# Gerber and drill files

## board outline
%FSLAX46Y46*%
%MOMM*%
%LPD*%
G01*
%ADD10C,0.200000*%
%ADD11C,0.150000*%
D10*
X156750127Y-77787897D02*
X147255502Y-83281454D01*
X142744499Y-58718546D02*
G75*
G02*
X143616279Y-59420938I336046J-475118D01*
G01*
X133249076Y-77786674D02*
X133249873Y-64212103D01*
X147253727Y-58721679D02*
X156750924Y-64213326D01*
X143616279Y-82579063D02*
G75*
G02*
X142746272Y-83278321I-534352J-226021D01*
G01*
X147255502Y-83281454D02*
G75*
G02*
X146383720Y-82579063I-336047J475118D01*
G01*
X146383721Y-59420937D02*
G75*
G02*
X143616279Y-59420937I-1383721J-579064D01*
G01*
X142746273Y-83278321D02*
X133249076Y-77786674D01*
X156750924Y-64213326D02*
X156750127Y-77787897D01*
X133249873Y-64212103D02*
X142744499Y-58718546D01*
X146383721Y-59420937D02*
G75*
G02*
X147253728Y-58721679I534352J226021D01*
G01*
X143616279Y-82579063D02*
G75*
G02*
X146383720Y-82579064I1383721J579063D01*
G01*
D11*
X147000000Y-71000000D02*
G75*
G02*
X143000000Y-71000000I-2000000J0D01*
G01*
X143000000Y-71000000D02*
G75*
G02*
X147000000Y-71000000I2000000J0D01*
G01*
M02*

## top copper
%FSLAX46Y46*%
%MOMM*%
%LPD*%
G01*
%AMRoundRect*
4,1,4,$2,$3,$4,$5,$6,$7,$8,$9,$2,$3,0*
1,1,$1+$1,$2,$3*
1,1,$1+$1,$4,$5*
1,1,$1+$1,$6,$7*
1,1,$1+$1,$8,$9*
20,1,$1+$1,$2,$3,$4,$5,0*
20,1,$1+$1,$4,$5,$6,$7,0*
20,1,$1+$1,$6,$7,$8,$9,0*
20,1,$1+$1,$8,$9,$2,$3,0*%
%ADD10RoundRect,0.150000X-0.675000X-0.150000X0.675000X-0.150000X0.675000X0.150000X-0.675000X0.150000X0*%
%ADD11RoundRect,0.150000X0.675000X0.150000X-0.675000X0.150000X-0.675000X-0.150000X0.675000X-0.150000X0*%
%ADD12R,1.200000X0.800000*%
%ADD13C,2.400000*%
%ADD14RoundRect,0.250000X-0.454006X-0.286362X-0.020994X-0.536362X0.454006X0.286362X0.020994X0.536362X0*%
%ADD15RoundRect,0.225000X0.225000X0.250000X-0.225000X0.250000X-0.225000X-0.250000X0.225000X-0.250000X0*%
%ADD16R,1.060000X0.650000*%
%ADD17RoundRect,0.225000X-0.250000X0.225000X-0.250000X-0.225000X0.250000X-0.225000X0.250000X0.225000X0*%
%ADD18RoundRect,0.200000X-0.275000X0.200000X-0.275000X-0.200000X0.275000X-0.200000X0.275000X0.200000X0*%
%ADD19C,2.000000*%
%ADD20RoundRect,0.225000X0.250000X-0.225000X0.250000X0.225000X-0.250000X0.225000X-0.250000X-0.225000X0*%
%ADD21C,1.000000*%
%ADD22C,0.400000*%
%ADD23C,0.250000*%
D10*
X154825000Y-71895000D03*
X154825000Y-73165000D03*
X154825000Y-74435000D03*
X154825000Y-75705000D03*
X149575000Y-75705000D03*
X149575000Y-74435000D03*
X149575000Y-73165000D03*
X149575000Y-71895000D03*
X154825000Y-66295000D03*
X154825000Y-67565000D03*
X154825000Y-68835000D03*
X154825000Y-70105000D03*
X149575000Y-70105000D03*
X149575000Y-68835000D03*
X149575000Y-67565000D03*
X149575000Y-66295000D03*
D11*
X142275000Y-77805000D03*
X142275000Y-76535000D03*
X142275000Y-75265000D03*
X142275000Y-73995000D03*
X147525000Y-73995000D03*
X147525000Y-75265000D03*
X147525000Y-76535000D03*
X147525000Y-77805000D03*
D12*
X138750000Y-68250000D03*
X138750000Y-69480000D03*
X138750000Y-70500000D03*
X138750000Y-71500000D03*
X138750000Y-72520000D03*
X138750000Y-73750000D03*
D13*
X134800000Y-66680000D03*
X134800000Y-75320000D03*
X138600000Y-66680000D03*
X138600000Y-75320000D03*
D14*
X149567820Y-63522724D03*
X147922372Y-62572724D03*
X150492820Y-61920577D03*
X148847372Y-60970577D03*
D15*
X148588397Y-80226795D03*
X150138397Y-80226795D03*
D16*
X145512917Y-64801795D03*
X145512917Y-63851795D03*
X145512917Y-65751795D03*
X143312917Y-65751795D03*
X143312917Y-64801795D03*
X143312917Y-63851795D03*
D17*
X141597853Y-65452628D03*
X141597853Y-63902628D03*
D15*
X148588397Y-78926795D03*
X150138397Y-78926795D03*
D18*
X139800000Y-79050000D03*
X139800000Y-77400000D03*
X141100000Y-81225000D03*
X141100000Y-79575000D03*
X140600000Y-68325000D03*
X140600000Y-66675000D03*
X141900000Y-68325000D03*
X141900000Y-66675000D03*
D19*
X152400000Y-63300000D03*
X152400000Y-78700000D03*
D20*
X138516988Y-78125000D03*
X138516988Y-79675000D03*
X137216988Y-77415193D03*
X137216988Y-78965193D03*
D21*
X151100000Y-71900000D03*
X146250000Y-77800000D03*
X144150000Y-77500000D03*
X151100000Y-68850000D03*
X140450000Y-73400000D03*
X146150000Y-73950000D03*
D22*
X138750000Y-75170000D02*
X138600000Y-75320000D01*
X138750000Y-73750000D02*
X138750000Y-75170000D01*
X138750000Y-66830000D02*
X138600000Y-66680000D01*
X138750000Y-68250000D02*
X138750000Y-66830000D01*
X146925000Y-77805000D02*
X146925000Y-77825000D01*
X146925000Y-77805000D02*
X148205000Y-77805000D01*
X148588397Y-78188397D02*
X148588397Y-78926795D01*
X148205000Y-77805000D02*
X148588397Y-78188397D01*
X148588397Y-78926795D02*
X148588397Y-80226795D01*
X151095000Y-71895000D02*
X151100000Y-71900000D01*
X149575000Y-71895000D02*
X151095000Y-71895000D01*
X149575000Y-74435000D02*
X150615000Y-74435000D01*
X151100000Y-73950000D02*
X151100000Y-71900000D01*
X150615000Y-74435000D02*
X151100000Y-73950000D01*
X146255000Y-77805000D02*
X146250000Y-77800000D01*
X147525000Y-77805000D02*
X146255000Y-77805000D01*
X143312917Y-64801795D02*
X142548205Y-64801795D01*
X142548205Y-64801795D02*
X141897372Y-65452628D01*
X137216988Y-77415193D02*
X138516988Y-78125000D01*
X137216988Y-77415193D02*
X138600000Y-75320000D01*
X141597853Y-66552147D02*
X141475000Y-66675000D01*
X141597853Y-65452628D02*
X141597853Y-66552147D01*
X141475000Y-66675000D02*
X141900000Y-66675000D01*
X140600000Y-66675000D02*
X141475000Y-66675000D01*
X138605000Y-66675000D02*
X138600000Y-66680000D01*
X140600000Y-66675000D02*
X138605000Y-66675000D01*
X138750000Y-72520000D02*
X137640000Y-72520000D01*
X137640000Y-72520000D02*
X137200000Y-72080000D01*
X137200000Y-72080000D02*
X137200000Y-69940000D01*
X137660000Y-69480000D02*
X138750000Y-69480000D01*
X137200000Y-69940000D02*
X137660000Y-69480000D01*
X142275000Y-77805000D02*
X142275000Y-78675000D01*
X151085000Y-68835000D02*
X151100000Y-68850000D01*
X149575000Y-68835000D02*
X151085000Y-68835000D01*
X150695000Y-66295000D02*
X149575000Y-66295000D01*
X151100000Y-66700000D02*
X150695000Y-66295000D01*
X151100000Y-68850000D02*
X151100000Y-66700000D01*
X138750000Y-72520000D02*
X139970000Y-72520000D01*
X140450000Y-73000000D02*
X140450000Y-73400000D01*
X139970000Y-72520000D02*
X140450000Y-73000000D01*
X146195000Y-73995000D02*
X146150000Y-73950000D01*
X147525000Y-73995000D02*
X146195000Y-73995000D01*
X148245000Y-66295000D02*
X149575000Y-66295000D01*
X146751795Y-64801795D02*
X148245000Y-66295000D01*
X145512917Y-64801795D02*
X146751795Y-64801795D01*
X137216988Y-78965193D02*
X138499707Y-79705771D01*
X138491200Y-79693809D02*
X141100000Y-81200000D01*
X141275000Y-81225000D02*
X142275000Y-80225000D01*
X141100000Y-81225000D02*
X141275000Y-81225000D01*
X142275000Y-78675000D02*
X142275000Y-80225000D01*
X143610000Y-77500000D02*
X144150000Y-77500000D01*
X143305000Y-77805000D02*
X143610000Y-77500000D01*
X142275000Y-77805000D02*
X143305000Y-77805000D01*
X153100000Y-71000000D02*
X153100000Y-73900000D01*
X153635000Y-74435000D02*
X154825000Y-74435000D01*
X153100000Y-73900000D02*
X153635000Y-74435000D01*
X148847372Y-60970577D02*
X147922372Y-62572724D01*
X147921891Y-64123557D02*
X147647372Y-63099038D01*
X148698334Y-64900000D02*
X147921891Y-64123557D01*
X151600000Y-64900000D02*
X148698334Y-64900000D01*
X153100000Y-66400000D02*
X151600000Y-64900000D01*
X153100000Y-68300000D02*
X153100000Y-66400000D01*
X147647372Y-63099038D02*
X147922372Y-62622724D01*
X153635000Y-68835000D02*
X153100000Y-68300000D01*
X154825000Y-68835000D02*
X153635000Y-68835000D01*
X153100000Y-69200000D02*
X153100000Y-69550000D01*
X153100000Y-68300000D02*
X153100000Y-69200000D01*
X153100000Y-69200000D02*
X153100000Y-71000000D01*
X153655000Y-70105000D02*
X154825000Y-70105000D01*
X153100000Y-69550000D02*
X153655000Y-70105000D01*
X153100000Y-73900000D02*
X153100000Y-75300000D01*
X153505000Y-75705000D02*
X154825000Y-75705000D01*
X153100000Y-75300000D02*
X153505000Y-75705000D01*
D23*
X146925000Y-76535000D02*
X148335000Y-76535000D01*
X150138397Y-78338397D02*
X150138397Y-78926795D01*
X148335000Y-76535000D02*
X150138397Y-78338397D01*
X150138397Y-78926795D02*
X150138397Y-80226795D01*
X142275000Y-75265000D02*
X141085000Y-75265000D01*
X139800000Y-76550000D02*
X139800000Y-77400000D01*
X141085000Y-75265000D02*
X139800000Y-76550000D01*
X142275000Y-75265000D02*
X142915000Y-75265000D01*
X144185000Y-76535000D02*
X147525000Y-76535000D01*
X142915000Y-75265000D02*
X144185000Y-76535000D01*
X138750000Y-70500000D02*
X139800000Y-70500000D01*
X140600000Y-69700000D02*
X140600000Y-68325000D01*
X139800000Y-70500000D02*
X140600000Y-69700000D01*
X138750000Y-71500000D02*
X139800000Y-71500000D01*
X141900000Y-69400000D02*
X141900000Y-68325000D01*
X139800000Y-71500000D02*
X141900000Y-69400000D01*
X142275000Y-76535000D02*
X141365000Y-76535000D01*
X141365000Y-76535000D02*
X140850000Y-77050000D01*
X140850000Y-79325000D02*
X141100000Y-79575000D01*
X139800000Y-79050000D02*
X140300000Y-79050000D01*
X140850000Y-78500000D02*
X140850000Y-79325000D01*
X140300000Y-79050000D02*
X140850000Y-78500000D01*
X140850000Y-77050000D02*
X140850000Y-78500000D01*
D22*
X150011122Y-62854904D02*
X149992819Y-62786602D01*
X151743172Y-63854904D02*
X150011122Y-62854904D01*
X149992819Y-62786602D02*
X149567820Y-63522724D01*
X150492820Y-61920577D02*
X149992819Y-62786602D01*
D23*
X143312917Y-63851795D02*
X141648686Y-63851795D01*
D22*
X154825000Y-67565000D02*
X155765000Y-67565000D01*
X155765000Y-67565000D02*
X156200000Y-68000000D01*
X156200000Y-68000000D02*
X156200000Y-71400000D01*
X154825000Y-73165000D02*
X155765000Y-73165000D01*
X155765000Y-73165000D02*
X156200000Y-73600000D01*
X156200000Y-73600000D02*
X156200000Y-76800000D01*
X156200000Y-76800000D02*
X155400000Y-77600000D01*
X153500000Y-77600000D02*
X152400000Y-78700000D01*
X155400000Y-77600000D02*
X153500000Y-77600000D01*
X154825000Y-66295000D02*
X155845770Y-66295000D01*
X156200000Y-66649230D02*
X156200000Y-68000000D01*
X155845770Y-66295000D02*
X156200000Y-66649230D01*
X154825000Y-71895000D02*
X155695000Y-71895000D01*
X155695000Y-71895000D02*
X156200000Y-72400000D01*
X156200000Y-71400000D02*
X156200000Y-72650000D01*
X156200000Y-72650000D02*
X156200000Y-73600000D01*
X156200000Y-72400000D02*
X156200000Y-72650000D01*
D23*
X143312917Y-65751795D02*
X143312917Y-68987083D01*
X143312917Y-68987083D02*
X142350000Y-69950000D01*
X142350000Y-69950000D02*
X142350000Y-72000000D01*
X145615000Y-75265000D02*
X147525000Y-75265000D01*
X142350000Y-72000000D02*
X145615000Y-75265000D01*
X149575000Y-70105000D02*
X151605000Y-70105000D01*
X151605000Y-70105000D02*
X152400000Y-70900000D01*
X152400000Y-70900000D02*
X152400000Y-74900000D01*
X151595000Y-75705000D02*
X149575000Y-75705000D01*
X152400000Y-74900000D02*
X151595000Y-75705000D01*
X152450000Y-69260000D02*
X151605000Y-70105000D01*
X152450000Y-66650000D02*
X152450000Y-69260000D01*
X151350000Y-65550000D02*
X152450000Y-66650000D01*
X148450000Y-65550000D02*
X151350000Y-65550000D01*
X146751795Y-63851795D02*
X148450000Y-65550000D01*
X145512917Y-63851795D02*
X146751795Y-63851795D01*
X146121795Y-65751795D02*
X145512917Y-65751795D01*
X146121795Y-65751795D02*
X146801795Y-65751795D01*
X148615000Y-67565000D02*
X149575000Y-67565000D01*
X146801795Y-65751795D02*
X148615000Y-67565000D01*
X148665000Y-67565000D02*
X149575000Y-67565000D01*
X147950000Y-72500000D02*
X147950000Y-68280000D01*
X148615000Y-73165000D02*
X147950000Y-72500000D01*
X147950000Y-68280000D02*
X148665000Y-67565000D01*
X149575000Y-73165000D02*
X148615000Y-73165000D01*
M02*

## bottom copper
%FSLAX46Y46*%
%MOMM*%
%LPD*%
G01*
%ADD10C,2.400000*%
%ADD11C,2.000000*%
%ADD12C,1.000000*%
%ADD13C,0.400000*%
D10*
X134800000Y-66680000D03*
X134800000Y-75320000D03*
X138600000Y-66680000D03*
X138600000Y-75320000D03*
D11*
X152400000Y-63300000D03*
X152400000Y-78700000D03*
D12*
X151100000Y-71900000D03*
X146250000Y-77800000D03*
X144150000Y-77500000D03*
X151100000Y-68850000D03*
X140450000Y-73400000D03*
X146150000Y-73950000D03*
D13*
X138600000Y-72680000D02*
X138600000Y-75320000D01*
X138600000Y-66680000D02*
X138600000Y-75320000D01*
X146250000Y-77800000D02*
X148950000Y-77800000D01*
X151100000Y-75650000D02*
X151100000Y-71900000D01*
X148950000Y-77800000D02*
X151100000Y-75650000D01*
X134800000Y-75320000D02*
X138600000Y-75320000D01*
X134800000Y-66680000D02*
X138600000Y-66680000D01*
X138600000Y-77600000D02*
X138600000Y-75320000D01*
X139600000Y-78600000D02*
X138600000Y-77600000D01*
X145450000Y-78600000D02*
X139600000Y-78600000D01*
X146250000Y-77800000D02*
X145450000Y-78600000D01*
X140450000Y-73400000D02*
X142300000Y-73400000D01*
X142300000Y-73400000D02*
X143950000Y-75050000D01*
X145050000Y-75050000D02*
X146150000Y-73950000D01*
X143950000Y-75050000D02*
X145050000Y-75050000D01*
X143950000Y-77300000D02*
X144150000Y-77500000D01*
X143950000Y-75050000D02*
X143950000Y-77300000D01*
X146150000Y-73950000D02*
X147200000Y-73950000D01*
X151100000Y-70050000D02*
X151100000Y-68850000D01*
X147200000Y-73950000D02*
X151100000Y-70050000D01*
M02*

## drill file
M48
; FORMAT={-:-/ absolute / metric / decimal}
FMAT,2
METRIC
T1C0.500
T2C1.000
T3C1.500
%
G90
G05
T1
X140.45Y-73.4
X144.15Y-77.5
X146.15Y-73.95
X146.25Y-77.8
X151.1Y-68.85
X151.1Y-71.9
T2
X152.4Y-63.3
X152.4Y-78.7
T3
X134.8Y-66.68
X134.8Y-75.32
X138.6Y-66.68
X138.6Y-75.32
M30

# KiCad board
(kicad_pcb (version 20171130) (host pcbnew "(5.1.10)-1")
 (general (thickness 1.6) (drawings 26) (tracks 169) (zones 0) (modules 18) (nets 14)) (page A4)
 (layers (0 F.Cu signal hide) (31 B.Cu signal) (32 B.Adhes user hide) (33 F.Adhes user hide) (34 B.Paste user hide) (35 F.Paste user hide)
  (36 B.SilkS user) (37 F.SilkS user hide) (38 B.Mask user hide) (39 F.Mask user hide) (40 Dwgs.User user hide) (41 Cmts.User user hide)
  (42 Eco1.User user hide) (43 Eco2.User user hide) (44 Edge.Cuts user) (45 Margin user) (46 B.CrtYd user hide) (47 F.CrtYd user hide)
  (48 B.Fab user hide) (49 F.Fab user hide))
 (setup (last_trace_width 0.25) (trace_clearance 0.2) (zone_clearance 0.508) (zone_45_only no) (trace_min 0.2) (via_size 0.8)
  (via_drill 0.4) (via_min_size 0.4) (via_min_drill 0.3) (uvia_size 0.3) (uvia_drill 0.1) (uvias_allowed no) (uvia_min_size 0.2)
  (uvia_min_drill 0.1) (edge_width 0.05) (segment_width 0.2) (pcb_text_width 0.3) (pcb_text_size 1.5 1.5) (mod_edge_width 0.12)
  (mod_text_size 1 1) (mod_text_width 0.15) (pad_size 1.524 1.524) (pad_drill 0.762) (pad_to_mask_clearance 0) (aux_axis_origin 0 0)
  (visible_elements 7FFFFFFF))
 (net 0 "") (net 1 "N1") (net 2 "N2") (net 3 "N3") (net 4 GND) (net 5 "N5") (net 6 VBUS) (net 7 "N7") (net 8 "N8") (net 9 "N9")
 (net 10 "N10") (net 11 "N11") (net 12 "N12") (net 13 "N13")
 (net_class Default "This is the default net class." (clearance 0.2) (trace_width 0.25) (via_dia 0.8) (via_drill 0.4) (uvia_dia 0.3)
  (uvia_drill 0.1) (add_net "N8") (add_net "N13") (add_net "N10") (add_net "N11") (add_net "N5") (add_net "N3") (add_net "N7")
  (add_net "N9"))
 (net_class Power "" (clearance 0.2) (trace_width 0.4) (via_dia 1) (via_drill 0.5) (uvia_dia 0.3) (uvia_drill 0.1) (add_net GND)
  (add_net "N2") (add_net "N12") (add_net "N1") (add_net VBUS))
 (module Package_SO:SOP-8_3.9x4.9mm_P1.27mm (layer F.Cu) (at 152.2 73.8)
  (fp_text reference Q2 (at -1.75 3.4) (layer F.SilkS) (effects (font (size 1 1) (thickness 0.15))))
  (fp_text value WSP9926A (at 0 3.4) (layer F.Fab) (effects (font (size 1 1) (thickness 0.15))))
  (pad 8 smd roundrect (at 2.625 -1.905) (size 1.65 0.6) (layers F.Cu F.Paste F.Mask) (roundrect_rratio 0.25) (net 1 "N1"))
  (pad 7 smd roundrect (at 2.625 -0.635) (size 1.65 0.6) (layers F.Cu F.Paste F.Mask) (roundrect_rratio 0.25) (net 1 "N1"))
  (pad 6 smd roundrect (at 2.625 0.635) (size 1.65 0.6) (layers F.Cu F.Paste F.Mask) (roundrect_rratio 0.25) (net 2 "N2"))
  (pad 5 smd roundrect (at 2.625 1.905) (size 1.65 0.6) (layers F.Cu F.Paste F.Mask) (roundrect_rratio 0.25) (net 2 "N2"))
  (pad 4 smd roundrect (at -2.625 1.905) (size 1.65 0.6) (layers F.Cu F.Paste F.Mask) (roundrect_rratio 0.25) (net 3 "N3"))
  (pad 3 smd roundrect (at -2.625 0.635) (size 1.65 0.6) (layers F.Cu F.Paste F.Mask) (roundrect_rratio 0.25) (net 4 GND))
  (pad 2 smd roundrect (at -2.625 -0.635) (size 1.65 0.6) (layers F.Cu F.Paste F.Mask) (roundrect_rratio 0.25) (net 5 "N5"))
  (pad 1 smd roundrect (at -2.625 -1.905) (size 1.65 0.6) (layers F.Cu F.Paste F.Mask) (roundrect_rratio 0.25) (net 4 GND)))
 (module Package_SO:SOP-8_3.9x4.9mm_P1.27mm (layer F.Cu) (at 152.2 68.2)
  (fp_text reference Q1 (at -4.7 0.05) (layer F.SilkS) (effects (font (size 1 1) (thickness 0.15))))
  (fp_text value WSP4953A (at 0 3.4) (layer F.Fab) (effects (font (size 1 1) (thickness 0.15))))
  (pad 8 smd roundrect (at 2.625 -1.905) (size 1.65 0.6) (layers F.Cu F.Paste F.Mask) (roundrect_rratio 0.25) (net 1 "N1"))
  (pad 7 smd roundrect (at 2.625 -0.635) (size 1.65 0.6) (layers F.Cu F.Paste F.Mask) (roundrect_rratio 0.25) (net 1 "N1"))
  (pad 6 smd roundrect (at 2.625 0.635) (size 1.65 0.6) (layers F.Cu F.Paste F.Mask) (roundrect_rratio 0.25) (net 2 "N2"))
  (pad 5 smd roundrect (at 2.625 1.905) (size 1.65 0.6) (layers F.Cu F.Paste F.Mask) (roundrect_rratio 0.25) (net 2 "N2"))
  (pad 4 smd roundrect (at -2.625 1.905) (size 1.65 0.6) (layers F.Cu F.Paste F.Mask) (roundrect_rratio 0.25) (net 3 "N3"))
  (pad 3 smd roundrect (at -2.625 0.635) (size 1.65 0.6) (layers F.Cu F.Paste F.Mask) (roundrect_rratio 0.25) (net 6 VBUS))
  (pad 2 smd roundrect (at -2.625 -0.635) (size 1.65 0.6) (layers F.Cu F.Paste F.Mask) (roundrect_rratio 0.25) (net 5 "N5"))
  (pad 1 smd roundrect (at -2.625 -1.905) (size 1.65 0.6) (layers F.Cu F.Paste F.Mask) (roundrect_rratio 0.25) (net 6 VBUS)))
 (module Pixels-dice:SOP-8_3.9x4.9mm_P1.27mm (layer F.Cu) (at 144.9 75.9 180)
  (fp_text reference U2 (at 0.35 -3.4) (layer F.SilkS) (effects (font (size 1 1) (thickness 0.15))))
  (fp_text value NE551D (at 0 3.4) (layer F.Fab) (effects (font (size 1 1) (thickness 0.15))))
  (pad 8 smd roundrect (at 2.625 -1.905 180) (size 1.65 0.6) (layers F.Cu F.Paste F.Mask) (roundrect_rratio 0.25) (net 6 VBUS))
  (pad 7 smd roundrect (at 2.625 -0.635 180) (size 1.65 0.6) (layers F.Cu F.Paste F.Mask) (roundrect_rratio 0.25) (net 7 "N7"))
  (pad 6 smd roundrect (at 2.625 0.635 180) (size 1.65 0.6) (layers F.Cu F.Paste F.Mask) (roundrect_rratio 0.25) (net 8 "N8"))
  (pad 5 smd roundrect (at 2.625 1.905 180) (size 1.65 0.6) (layers F.Cu F.Paste F.Mask) (roundrect_rratio 0.25))
  (pad 4 smd roundrect (at -2.625 1.905 180) (size 1.65 0.6) (layers F.Cu F.Paste F.Mask) (roundrect_rratio 0.25) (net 6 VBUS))
  (pad 3 smd roundrect (at -2.625 0.635 180) (size 1.65 0.6) (layers F.Cu F.Paste F.Mask) (roundrect_rratio 0.25) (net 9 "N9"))
  (pad 2 smd roundrect (at -2.625 -0.635 180) (size 1.65 0.6) (layers F.Cu F.Paste F.Mask) (roundrect_rratio 0.25) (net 8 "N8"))
  (pad 1 smd roundrect (at -2.625 -1.905 180) (size 1.65 0.6) (layers F.Cu F.Paste F.Mask) (roundrect_rratio 0.25) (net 4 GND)))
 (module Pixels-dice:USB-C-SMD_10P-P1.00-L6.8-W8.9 (layer F.Cu) (at 136.7 71)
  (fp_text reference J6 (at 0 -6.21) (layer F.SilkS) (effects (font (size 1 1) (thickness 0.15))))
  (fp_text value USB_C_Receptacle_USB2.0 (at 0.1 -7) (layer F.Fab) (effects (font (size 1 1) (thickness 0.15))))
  (pad B12 smd rect (at 2.05 -2.75 270) (size 0.8 1.2) (layers F.Cu F.Paste F.Mask) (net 4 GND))
  (pad B9 smd rect (at 2.05 -1.52 270) (size 0.8 1.2) (layers F.Cu F.Paste F.Mask) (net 6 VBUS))
  (pad A5 smd rect (at 2.05 -0.5 270) (size 0.8 1.2) (layers F.Cu F.Paste F.Mask) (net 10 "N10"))
  (pad B5 smd rect (at 2.05 0.5 270) (size 0.8 1.2) (layers F.Cu F.Paste F.Mask) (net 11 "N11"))
  (pad A9 smd rect (at 2.05 1.52 270) (size 0.8 1.2) (layers F.Cu F.Paste F.Mask) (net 6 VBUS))
  (pad A12 smd rect (at 2.05 2.75 270) (size 0.8 1.2) (layers F.Cu F.Paste F.Mask) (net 4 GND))
  (pad S1 thru_hole circle (at -1.9 -4.32 270) (size 2.4 2.4) (drill 1.5) (layers *.Cu *.Mask) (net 4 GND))
  (pad S1 thru_hole circle (at -1.9 4.32 270) (size 2.4 2.4) (drill 1.5) (layers *.Cu *.Mask) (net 4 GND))
  (pad S1 thru_hole circle (at 1.9 -4.32 270) (size 2.4 2.4) (drill 1.5) (layers *.Cu *.Mask) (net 4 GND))
  (pad S1 thru_hole circle (at 1.9 4.32 270) (size 2.4 2.4) (drill 1.5) (layers *.Cu *.Mask) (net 4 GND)))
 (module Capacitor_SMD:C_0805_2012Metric (layer F.Cu) (at 148.745096 63.047724 330)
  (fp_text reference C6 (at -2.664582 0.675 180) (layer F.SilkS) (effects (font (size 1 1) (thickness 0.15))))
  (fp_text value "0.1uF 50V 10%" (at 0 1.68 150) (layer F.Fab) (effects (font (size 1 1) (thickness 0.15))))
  (pad 2 smd roundrect (at 0.95 0 330) (size 1 1.45) (layers F.Cu F.Paste F.Mask) (roundrect_rratio 0.25) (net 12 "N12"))
  (pad 1 smd roundrect (at -0.95 0 330) (size 1 1.45) (layers F.Cu F.Paste F.Mask) (roundrect_rratio 0.25) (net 2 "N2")))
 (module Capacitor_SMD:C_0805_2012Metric (layer F.Cu) (at 149.670096 61.445577 330)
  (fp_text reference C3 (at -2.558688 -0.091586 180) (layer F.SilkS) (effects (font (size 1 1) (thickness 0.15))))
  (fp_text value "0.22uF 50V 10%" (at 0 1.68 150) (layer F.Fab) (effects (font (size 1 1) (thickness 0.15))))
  (pad 2 smd roundrect (at 0.95 0 330) (size 1 1.45) (layers F.Cu F.Paste F.Mask) (roundrect_rratio 0.25) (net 12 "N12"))
  (pad 1 smd roundrect (at -0.95 0 330) (size 1 1.45) (layers F.Cu F.Paste F.Mask) (roundrect_rratio 0.25) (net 2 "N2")))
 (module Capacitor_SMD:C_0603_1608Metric (layer F.Cu) (at 149.363397 80.226795 180)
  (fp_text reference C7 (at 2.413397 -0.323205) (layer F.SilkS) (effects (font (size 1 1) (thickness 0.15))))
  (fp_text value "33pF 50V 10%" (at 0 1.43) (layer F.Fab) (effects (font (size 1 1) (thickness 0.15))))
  (pad 2 smd roundrect (at 0.775 0 180) (size 0.9 0.95) (layers F.Cu F.Paste F.Mask) (roundrect_rratio 0.25) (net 4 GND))
  (pad 1 smd roundrect (at -0.775 0 180) (size 0.9 0.95) (layers F.Cu F.Paste F.Mask) (roundrect_rratio 0.25) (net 8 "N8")))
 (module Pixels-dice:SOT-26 (layer F.Cu) (at 144.412917 64.801795 180)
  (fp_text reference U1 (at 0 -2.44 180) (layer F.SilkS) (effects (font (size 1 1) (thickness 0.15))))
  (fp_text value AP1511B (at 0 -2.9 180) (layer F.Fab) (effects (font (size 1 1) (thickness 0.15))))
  (pad 5 smd rect (at -1.1 0) (size 1.06 0.65) (layers F.Cu F.Paste F.Mask) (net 6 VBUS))
  (pad 6 smd rect (at -1.1 0.95) (size 1.06 0.65) (layers F.Cu F.Paste F.Mask) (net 3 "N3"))
  (pad 4 smd rect (at -1.1 -0.95) (size 1.06 0.65) (layers F.Cu F.Paste F.Mask) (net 5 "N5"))
  (pad 3 smd rect (at 1.1 -0.95) (size 1.06 0.65) (layers F.Cu F.Paste F.Mask) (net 9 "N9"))
  (pad 2 smd rect (at 1.1 0) (size 1.06 0.65) (layers F.Cu F.Paste F.Mask) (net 4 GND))
  (pad 1 smd rect (at 1.1 0.95) (size 1.06 0.65) (layers F.Cu F.Paste F.Mask) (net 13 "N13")))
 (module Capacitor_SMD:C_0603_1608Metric (layer F.Cu) (at 141.597853 64.677628 270)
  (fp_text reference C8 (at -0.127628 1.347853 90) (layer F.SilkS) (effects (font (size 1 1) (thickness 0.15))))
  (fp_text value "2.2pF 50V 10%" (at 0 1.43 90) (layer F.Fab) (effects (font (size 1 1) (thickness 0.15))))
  (pad 2 smd roundrect (at 0.775 0 270) (size 0.9 0.95) (layers F.Cu F.Paste F.Mask) (roundrect_rratio 0.25) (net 4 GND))
  (pad 1 smd roundrect (at -0.775 0 270) (size 0.9 0.95) (layers F.Cu F.Paste F.Mask) (roundrect_rratio 0.25) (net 13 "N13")))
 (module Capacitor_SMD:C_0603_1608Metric (layer F.Cu) (at 149.363397 78.926795 180)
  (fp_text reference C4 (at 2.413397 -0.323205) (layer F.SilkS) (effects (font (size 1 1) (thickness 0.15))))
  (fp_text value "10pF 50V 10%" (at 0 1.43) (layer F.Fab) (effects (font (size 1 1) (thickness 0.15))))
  (pad 2 smd roundrect (at 0.775 0 180) (size 0.9 0.95) (layers F.Cu F.Paste F.Mask) (roundrect_rratio 0.25) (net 4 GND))
  (pad 1 smd roundrect (at -0.775 0 180) (size 0.9 0.95) (layers F.Cu F.Paste F.Mask) (roundrect_rratio 0.25) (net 8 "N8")))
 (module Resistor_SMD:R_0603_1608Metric (layer F.Cu) (at 139.8 78.225 270)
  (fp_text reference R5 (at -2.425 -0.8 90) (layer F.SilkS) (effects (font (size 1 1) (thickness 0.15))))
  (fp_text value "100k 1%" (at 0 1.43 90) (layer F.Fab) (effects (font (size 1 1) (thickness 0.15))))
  (pad 2 smd roundrect (at 0.825 0 270) (size 0.8 0.95) (layers F.Cu F.Paste F.Mask) (roundrect_rratio 0.25) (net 7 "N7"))
  (pad 1 smd roundrect (at -0.825 0 270) (size 0.8 0.95) (layers F.Cu F.Paste F.Mask) (roundrect_rratio 0.25) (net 8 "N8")))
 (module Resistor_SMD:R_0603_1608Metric (layer F.Cu) (at 141.1 80.4 270)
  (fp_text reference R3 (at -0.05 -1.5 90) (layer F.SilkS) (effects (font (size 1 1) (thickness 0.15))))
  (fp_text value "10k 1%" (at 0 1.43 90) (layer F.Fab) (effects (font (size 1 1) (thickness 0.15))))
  (pad 2 smd roundrect (at 0.825 0 270) (size 0.8 0.95) (layers F.Cu F.Paste F.Mask) (roundrect_rratio 0.25) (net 6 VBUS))
  (pad 1 smd roundrect (at -0.825 0 270) (size 0.8 0.95) (layers F.Cu F.Paste F.Mask) (roundrect_rratio 0.25) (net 7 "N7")))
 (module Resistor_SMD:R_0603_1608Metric (layer F.Cu) (at 140.6 67.5 270)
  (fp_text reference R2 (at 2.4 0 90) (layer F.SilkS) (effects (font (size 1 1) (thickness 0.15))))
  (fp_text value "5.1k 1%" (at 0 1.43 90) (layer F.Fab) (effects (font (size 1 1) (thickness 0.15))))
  (pad 2 smd roundrect (at 0.825 0 270) (size 0.8 0.95) (layers F.Cu F.Paste F.Mask) (roundrect_rratio 0.25) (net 10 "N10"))
  (pad 1 smd roundrect (at -0.825 0 270) (size 0.8 0.95) (layers F.Cu F.Paste F.Mask) (roundrect_rratio 0.25) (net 4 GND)))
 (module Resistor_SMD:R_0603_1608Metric (layer F.Cu) (at 141.9 67.5 270)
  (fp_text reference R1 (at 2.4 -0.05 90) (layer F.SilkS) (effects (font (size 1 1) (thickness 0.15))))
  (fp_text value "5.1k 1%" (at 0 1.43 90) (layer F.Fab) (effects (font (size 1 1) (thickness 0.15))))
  (pad 2 smd roundrect (at 0.825 0 270) (size 0.8 0.95) (layers F.Cu F.Paste F.Mask) (roundrect_rratio 0.25) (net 11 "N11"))
  (pad 1 smd roundrect (at -0.825 0 270) (size 0.8 0.95) (layers F.Cu F.Paste F.Mask) (roundrect_rratio 0.25) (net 4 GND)))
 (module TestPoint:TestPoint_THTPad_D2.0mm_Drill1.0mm (layer F.Cu) (at 152.4 63.3)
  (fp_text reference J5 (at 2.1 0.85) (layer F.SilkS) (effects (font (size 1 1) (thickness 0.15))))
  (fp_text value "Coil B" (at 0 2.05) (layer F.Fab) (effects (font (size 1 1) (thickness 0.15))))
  (pad 1 thru_hole circle (at 0 0) (size 2 2) (drill 1) (layers *.Cu *.Mask) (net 12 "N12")))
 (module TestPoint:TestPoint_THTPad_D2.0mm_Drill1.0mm (layer F.Cu) (at 152.4 78.7)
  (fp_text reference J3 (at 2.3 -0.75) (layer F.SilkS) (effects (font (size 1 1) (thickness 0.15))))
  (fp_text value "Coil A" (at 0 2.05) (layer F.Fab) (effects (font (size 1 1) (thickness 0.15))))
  (pad 1 thru_hole circle (at 0 0) (size 2 2) (drill 1) (layers *.Cu *.Mask) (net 1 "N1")))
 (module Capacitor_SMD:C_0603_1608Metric (layer F.Cu) (at 138.516988 78.9 90)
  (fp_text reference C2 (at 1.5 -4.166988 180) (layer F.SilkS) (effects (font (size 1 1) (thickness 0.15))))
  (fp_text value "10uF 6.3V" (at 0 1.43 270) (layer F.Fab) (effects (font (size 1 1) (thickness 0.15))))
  (pad 2 smd roundrect (at 0.775 0 90) (size 0.9 0.95) (layers F.Cu F.Paste F.Mask) (roundrect_rratio 0.25) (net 4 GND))
  (pad 1 smd roundrect (at -0.775 0 90) (size 0.9 0.95) (layers F.Cu F.Paste F.Mask) (roundrect_rratio 0.25) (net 6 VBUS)))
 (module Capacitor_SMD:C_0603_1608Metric (layer F.Cu) (at 137.216988 78.190193 90)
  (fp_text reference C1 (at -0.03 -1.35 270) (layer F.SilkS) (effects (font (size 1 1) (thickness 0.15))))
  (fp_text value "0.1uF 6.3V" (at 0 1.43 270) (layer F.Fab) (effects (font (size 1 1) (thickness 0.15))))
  (pad 2 smd roundrect (at 0.775 0 90) (size 0.9 0.95) (layers F.Cu F.Paste F.Mask) (roundrect_rratio 0.25) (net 4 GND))
  (pad 1 smd roundrect (at -0.775 0 90) (size 0.9 0.95) (layers F.Cu F.Paste F.Mask) (roundrect_rratio 0.25) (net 6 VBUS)))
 (gr_line (start 156.750127 77.787897) (end 147.255502 83.281454) (layer Edge.Cuts) (width 0.2))
 (gr_arc (start 143.080545 59.193664) (end 142.744499 58.718546) (angle 148.2594298) (layer Edge.Cuts) (width 0.2))
 (gr_line (start 133.249076 77.786674) (end 133.249873 64.212103) (layer Edge.Cuts) (width 0.2))
 (gr_line (start 147.253727 58.721679) (end 156.750924 64.213326) (layer Edge.Cuts) (width 0.2))
 (gr_arc (start 143.081927 82.805084) (end 143.616279 82.579063) (angle 148.274571) (layer Edge.Cuts) (width 0.2))
 (gr_arc (start 146.919455 82.806336) (end 147.255502 83.281454) (angle 148.2594298) (layer Edge.Cuts) (width 0.2))
 (gr_arc (start 145 60.000001) (end 146.383721 59.420937) (angle 225.4169665) (layer Edge.Cuts) (width 0.2))
 (gr_line (start 142.746273 83.278321) (end 133.249076 77.786674) (layer Edge.Cuts) (width 0.2))
 (gr_line (start 156.750924 64.213326) (end 156.750127 77.787897) (layer Edge.Cuts) (width 0.2))
 (gr_line (start 133.249873 64.212103) (end 142.744499 58.718546) (layer Edge.Cuts) (width 0.2))
 (gr_arc (start 146.918073 59.194916) (end 146.383721 59.420937) (angle 148.274571) (layer Edge.Cuts) (width 0.2))
 (gr_arc (start 145 82) (end 143.616279 82.579063) (angle 225.4169665) (layer Edge.Cuts) (width 0.2))
 (gr_circle (center 145 71) (end 147 71) (layer Edge.Cuts) (width 0.15))
 (segment (start 138.75 75.17) (end 138.6 75.32) (width 0.4) (layer F.Cu) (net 4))
 (segment (start 138.75 73.75) (end 138.75 75.17) (width 0.4) (layer F.Cu) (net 4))
 (segment (start 138.75 66.83) (end 138.6 66.68) (width 0.4) (layer F.Cu) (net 4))
 (segment (start 138.75 68.25) (end 138.75 66.83) (width 0.4) (layer F.Cu) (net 4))
 (segment (start 138.6 72.68) (end 138.6 75.32) (width 0.4) (layer B.Cu) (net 4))
 (segment (start 138.6 66.68) (end 138.6 75.32) (width 0.4) (layer B.Cu) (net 4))
 (segment (start 146.925 77.805) (end 146.925 77.825) (width 0.4) (layer F.Cu) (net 4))
 (segment (start 146.925 77.805) (end 148.205 77.805) (width 0.4) (layer F.Cu) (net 4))
 (segment (start 148.588397 78.188397) (end 148.588397 78.926795) (width 0.4) (layer F.Cu) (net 4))
 (segment (start 148.205 77.805) (end 148.588397 78.188397) (width 0.4) (layer F.Cu) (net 4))
 (segment (start 148.588397 78.926795) (end 148.588397 80.226795) (width 0.4) (layer F.Cu) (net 4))
 (via (at 151.1 71.9) (size 1) (drill 0.5) (layers F.Cu B.Cu) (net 4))
 (segment (start 151.095 71.895) (end 151.1 71.9) (width 0.4) (layer F.Cu) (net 4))
 (segment (start 149.575 71.895) (end 151.095 71.895) (width 0.4) (layer F.Cu) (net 4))
 (segment (start 149.575 74.435) (end 150.615 74.435) (width 0.4) (layer F.Cu) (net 4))
 (segment (start 151.1 73.95) (end 151.1 71.9) (width 0.4) (layer F.Cu) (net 4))
 (segment (start 150.615 74.435) (end 151.1 73.95) (width 0.4) (layer F.Cu) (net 4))
 (via (at 146.25 77.8) (size 1) (drill 0.5) (layers F.Cu B.Cu) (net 4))
 (segment (start 146.255 77.805) (end 146.25 77.8) (width 0.4) (layer F.Cu) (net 4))
 (segment (start 147.525 77.805) (end 146.255 77.805) (width 0.4) (layer F.Cu) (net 4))
 (segment (start 143.312917 64.801795) (end 142.548205 64.801795) (width 0.4) (layer F.Cu) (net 4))
 (segment (start 142.548205 64.801795) (end 141.897372 65.452628) (width 0.4) (layer F.Cu) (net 4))
 (segment (start 137.216988 77.415193) (end 138.516988 78.125) (width 0.4) (layer F.Cu) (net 4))
 (segment (start 137.216988 77.415193) (end 138.6 75.32) (width 0.4) (layer F.Cu) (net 4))
 (segment (start 146.25 77.8) (end 148.95 77.8) (width 0.4) (layer B.Cu) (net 4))
 (segment (start 151.1 75.65) (end 151.1 71.9) (width 0.4) (layer B.Cu) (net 4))
 (segment (start 148.95 77.8) (end 151.1 75.65) (width 0.4) (layer B.Cu) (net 4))
 (segment (start 134.8 75.32) (end 138.6 75.32) (width 0.4) (layer B.Cu) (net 4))
 (segment (start 134.8 66.68) (end 138.6 66.68) (width 0.4) (layer B.Cu) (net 4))
 (segment (start 141.597853 66.552147) (end 141.475 66.675) (width 0.4) (layer F.Cu) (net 4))
 (segment (start 141.597853 65.452628) (end 141.597853 66.552147) (width 0.4) (layer F.Cu) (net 4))
 (segment (start 141.475 66.675) (end 141.9 66.675) (width 0.4) (layer F.Cu) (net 4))
 (segment (start 140.6 66.675) (end 141.475 66.675) (width 0.4) (layer F.Cu) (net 4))
 (segment (start 138.605 66.675) (end 138.6 66.68) (width 0.4) (layer F.Cu) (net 4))
 (segment (start 140.6 66.675) (end 138.605 66.675) (width 0.4) (layer F.Cu) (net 4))
 (segment (start 138.6 77.6) (end 138.6 75.32) (width 0.4) (layer B.Cu) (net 4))
 (segment (start 139.6 78.6) (end 138.6 77.6) (width 0.4) (layer B.Cu) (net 4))
 (segment (start 145.45 78.6) (end 139.6 78.6) (width 0.4) (layer B.Cu) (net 4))
 (segment (start 146.25 77.8) (end 145.45 78.6) (width 0.4) (layer B.Cu) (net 4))
 (segment (start 138.75 72.52) (end 137.64 72.52) (width 0.4) (layer F.Cu) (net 6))
 (segment (start 137.64 72.52) (end 137.2 72.08) (width 0.4) (layer F.Cu) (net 6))
 (segment (start 137.2 72.08) (end 137.2 69.94) (width 0.4) (layer F.Cu) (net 6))
 (segment (start 137.66 69.48) (end 138.75 69.48) (width 0.4) (layer F.Cu) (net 6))
 (segment (start 137.2 69.94) (end 137.66 69.48) (width 0.4) (layer F.Cu) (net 6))
 (via (at 144.15 77.5) (size 1) (drill 0.5) (layers F.Cu B.Cu) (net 6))
 (segment (start 142.275 77.805) (end 142.275 78.675) (width 0.4) (layer F.Cu) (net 6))
 (via (at 151.1 68.85) (size 1) (drill 0.5) (layers F.Cu B.Cu) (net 6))
 (segment (start 151.085 68.835) (end 151.1 68.85) (width 0.4) (layer F.Cu) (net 6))
 (segment (start 149.575 68.835) (end 151.085 68.835) (width 0.4) (layer F.Cu) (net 6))
 (segment (start 150.695 66.295) (end 149.575 66.295) (width 0.4) (layer F.Cu) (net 6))
 (segment (start 151.1 66.7) (end 150.695 66.295) (width 0.4) (layer F.Cu) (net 6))
 (segment (start 151.1 68.85) (end 151.1 66.7) (width 0.4) (layer F.Cu) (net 6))
 (segment (start 138.75 72.52) (end 139.97 72.52) (width 0.4) (layer F.Cu) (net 6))
 (via (at 140.45 73.4) (size 1) (drill 0.5) (layers F.Cu B.Cu) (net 6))
 (segment (start 140.45 73) (end 140.45 73.4) (width 0.4) (layer F.Cu) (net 6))
 (segment (start 139.97 72.52) (end 140.45 73) (width 0.4) (layer F.Cu) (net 6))
 (via (at 146.15 73.95) (size 1) (drill 0.5) (layers F.Cu B.Cu) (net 6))
 (segment (start 146.195 73.995) (end 146.15 73.95) (width 0.4) (layer F.Cu) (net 6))
 (segment (start 147.525 73.995) (end 146.195 73.995) (width 0.4) (layer F.Cu) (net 6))
 (segment (start 148.245 66.295) (end 149.575 66.295) (width 0.4) (layer F.Cu) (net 6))
 (segment (start 146.751795 64.801795) (end 148.245 66.295) (width 0.4) (layer F.Cu) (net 6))
 (segment (start 145.512917 64.801795) (end 146.751795 64.801795) (width 0.4) (layer F.Cu) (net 6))
 (segment (start 137.216988 78.965193) (end 138.499707 79.705771) (width 0.4) (layer F.Cu) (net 6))
 (segment (start 138.4912 79.693809) (end 141.1 81.2) (width 0.4) (layer F.Cu) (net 6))
 (segment (start 141.275 81.225) (end 142.275 80.225) (width 0.4) (layer F.Cu) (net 6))
 (segment (start 141.1 81.225) (end 141.275 81.225) (width 0.4) (layer F.Cu) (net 6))
 (segment (start 142.275 78.675) (end 142.275 80.225) (width 0.4) (layer F.Cu) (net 6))
 (segment (start 140.45 73.4) (end 142.3 73.4) (width 0.4) (layer B.Cu) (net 6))
 (segment (start 142.3 73.4) (end 143.95 75.05) (width 0.4) (layer B.Cu) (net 6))
 (segment (start 145.05 75.05) (end 146.15 73.95) (width 0.4) (layer B.Cu) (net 6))
 (segment (start 143.95 75.05) (end 145.05 75.05) (width 0.4) (layer B.Cu) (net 6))
 (segment (start 143.95 77.3) (end 144.15 77.5) (width 0.4) (layer B.Cu) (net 6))
 (segment (start 143.95 75.05) (end 143.95 77.3) (width 0.4) (layer B.Cu) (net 6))
 (segment (start 143.61 77.5) (end 144.15 77.5) (width 0.4) (layer F.Cu) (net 6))
 (segment (start 143.305 77.805) (end 143.61 77.5) (width 0.4) (layer F.Cu) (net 6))
 (segment (start 142.275 77.805) (end 143.305 77.805) (width 0.4) (layer F.Cu) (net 6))
 (segment (start 146.15 73.95) (end 147.2 73.95) (width 0.4) (layer B.Cu) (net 6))
 (segment (start 151.1 70.05) (end 151.1 68.85) (width 0.4) (layer B.Cu) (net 6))
 (segment (start 147.2 73.95) (end 151.1 70.05) (width 0.4) (layer B.Cu) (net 6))
 (segment (start 153.1 71) (end 153.1 73.9) (width 0.4) (layer F.Cu) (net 2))
 (segment (start 153.635 74.435) (end 154.825 74.435) (width 0.4) (layer F.Cu) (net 2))
 (segment (start 153.1 73.9) (end 153.635 74.435) (width 0.4) (layer F.Cu) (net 2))
 (segment (start 148.847372 60.970577) (end 147.922372 62.572724) (width 0.4) (layer F.Cu) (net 2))
 (segment (start 147.921891 64.123557) (end 147.647372 63.099038) (width 0.4) (layer F.Cu) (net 2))
 (segment (start 148.698334 64.9) (end 147.921891 64.123557) (width 0.4) (layer F.Cu) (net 2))
 (segment (start 151.6 64.9) (end 148.698334 64.9) (width 0.4) (layer F.Cu) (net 2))
 (segment (start 153.1 66.4) (end 151.6 64.9) (width 0.4) (layer F.Cu) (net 2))
 (segment (start 153.1 68.3) (end 153.1 66.4) (width 0.4) (layer F.Cu) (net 2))
 (segment (start 147.647372 63.099038) (end 147.922372 62.622724) (width 0.4) (layer F.Cu) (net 2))
 (segment (start 153.635 68.835) (end 153.1 68.3) (width 0.4) (layer F.Cu) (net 2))
 (segment (start 154.825 68.835) (end 153.635 68.835) (width 0.4) (layer F.Cu) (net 2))
 (segment (start 153.1 69.2) (end 153.1 69.55) (width 0.4) (layer F.Cu) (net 2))
 (segment (start 153.1 68.3) (end 153.1 69.2) (width 0.4) (layer F.Cu) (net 2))
 (segment (start 153.1 69.2) (end 153.1 71) (width 0.4) (layer F.Cu) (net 2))
 (segment (start 153.655 70.105) (end 154.825 70.105) (width 0.4) (layer F.Cu) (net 2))
 (segment (start 153.1 69.55) (end 153.655 70.105) (width 0.4) (layer F.Cu) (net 2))
 (segment (start 153.1 73.9) (end 153.1 75.3) (width 0.4) (layer F.Cu) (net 2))
 (segment (start 153.505 75.705) (end 154.825 75.705) (width 0.4) (layer F.Cu) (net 2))
 (segment (start 153.1 75.3) (end 153.505 75.705) (width 0.4) (layer F.Cu) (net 2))
 (segment (start 146.925 76.535) (end 148.335 76.535) (width 0.25) (layer F.Cu) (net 8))
 (segment (start 150.138397 78.338397) (end 150.138397 78.926795) (width 0.25) (layer F.Cu) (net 8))
 (segment (start 148.335 76.535) (end 150.138397 78.338397) (width 0.25) (layer F.Cu) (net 8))
 (segment (start 150.138397 78.926795) (end 150.138397 80.226795) (width 0.25) (layer F.Cu) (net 8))
 (segment (start 142.275 75.265) (end 141.085 75.265) (width 0.25) (layer F.Cu) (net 8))
 (segment (start 139.8 76.55) (end 139.8 77.4) (width 0.25) (layer F.Cu) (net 8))
 (segment (start 141.085 75.265) (end 139.8 76.55) (width 0.25) (layer F.Cu) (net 8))
 (segment (start 142.275 75.265) (end 142.915 75.265) (width 0.25) (layer F.Cu) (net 8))
 (segment (start 144.185 76.535) (end 147.525 76.535) (width 0.25) (layer F.Cu) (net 8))
 (segment (start 142.915 75.265) (end 144.185 76.535) (width 0.25) (layer F.Cu) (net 8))
 (segment (start 138.75 70.5) (end 139.8 70.5) (width 0.25) (layer F.Cu) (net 10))
 (segment (start 140.6 69.7) (end 140.6 68.325) (width 0.25) (layer F.Cu) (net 10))
 (segment (start 139.8 70.5) (end 140.6 69.7) (width 0.25) (layer F.Cu) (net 10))
 (segment (start 138.75 71.5) (end 139.8 71.5) (width 0.25) (layer F.Cu) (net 11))
 (segment (start 141.9 69.4) (end 141.9 68.325) (width 0.25) (layer F.Cu) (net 11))
 (segment (start 139.8 71.5) (end 141.9 69.4) (width 0.25) (layer F.Cu) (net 11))
 (segment (start 142.275 76.535) (end 141.365 76.535) (width 0.25) (layer F.Cu) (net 7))
 (segment (start 141.365 76.535) (end 140.85 77.05) (width 0.25) (layer F.Cu) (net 7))
 (segment (start 140.85 79.325) (end 141.1 79.575) (width 0.25) (layer F.Cu) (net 7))
 (segment (start 139.8 79.05) (end 140.3 79.05) (width 0.25) (layer F.Cu) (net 7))
 (segment (start 140.85 78.5) (end 140.85 79.325) (width 0.25) (layer F.Cu) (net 7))
 (segment (start 140.3 79.05) (end 140.85 78.5) (width 0.25) (layer F.Cu) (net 7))
 (segment (start 140.85 77.05) (end 140.85 78.5) (width 0.25) (layer F.Cu) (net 7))
 (segment (start 150.011122 62.854904) (end 149.992819 62.786602) (width 0.4) (layer F.Cu) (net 12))
 (segment (start 151.743172 63.854904) (end 150.011122 62.854904) (width 0.4) (layer F.Cu) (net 12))
 (segment (start 149.992819 62.786602) (end 149.56782 63.522724) (width 0.4) (layer F.Cu) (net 12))
 (segment (start 150.49282 61.920577) (end 149.992819 62.786602) (width 0.4) (layer F.Cu) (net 12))
 (segment (start 143.312917 63.851795) (end 141.648686 63.851795) (width 0.25) (layer F.Cu) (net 13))
 (segment (start 154.825 67.565) (end 155.765 67.565) (width 0.4) (layer F.Cu) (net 1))
 (segment (start 155.765 67.565) (end 156.2 68) (width 0.4) (layer F.Cu) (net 1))
 (segment (start 156.2 68) (end 156.2 71.4) (width 0.4) (layer F.Cu) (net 1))
 (segment (start 154.825 73.165) (end 155.765 73.165) (width 0.4) (layer F.Cu) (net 1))
 (segment (start 155.765 73.165) (end 156.2 73.6) (width 0.4) (layer F.Cu) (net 1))
 (segment (start 156.2 73.6) (end 156.2 76.8) (width 0.4) (layer F.Cu) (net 1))
 (segment (start 156.2 76.8) (end 155.4 77.6) (width 0.4) (layer F.Cu) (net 1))
 (segment (start 153.5 77.6) (end 152.4 78.7) (width 0.4) (layer F.Cu) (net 1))
 (segment (start 155.4 77.6) (end 153.5 77.6) (width 0.4) (layer F.Cu) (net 1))
 (segment (start 154.825 66.295) (end 155.84577 66.295) (width 0.4) (layer F.Cu) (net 1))
 (segment (start 156.2 66.64923) (end 156.2 68) (width 0.4) (layer F.Cu) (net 1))
 (segment (start 155.84577 66.295) (end 156.2 66.64923) (width 0.4) (layer F.Cu) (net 1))
 (segment (start 154.825 71.895) (end 155.695 71.895) (width 0.4) (layer F.Cu) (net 1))
 (segment (start 155.695 71.895) (end 156.2 72.4) (width 0.4) (layer F.Cu) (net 1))
 (segment (start 156.2 71.4) (end 156.2 72.65) (width 0.4) (layer F.Cu) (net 1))
 (segment (start 156.2 72.65) (end 156.2 73.6) (width 0.4) (layer F.Cu) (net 1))
 (segment (start 156.2 72.4) (end 156.2 72.65) (width 0.4) (layer F.Cu) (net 1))
 (segment (start 143.312917 65.751795) (end 143.312917 68.987083) (width 0.25) (layer F.Cu) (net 9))
 (segment (start 143.312917 68.987083) (end 142.35 69.95) (width 0.25) (layer F.Cu) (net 9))
 (segment (start 142.35 69.95) (end 142.35 72) (width 0.25) (layer F.Cu) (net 9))
 (segment (start 145.615 75.265) (end 147.525 75.265) (width 0.25) (layer F.Cu) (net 9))
 (segment (start 142.35 72) (end 145.615 75.265) (width 0.25) (layer F.Cu) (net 9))
 (segment (start 149.575 70.105) (end 151.605 70.105) (width 0.25) (layer F.Cu) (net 3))
 (segment (start 151.605 70.105) (end 152.4 70.9) (width 0.25) (layer F.Cu) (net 3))
 (segment (start 152.4 70.9) (end 152.4 74.9) (width 0.25) (layer F.Cu) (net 3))
 (segment (start 151.595 75.705) (end 149.575 75.705) (width 0.25) (layer F.Cu) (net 3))
 (segment (start 152.4 74.9) (end 151.595 75.705) (width 0.25) (layer F.Cu) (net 3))
 (segment (start 152.45 69.26) (end 151.605 70.105) (width 0.25) (layer F.Cu) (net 3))
 (segment (start 152.45 66.65) (end 152.45 69.26) (width 0.25) (layer F.Cu) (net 3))
 (segment (start 151.35 65.55) (end 152.45 66.65) (width 0.25) (layer F.Cu) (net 3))
 (segment (start 148.45 65.55) (end 151.35 65.55) (width 0.25) (layer F.Cu) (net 3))
 (segment (start 146.751795 63.851795) (end 148.45 65.55) (width 0.25) (layer F.Cu) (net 3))
 (segment (start 145.512917 63.851795) (end 146.751795 63.851795) (width 0.25) (layer F.Cu) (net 3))
 (segment (start 146.121795 65.751795) (end 145.512917 65.751795) (width 0.25) (layer F.Cu) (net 5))
 (segment (start 146.121795 65.751795) (end 146.801795 65.751795) (width 0.25) (layer F.Cu) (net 5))
 (segment (start 148.615 67.565) (end 149.575 67.565) (width 0.25) (layer F.Cu) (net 5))
 (segment (start 146.801795 65.751795) (end 148.615 67.565) (width 0.25) (layer F.Cu) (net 5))
 (segment (start 148.665 67.565) (end 149.575 67.565) (width 0.25) (layer F.Cu) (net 5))
 (segment (start 147.95 72.5) (end 147.95 68.28) (width 0.25) (layer F.Cu) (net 5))
 (segment (start 148.615 73.165) (end 147.95 72.5) (width 0.25) (layer F.Cu) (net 5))
 (segment (start 147.95 68.28) (end 148.665 67.565) (width 0.25) (layer F.Cu) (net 5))
 (segment (start 149.575 73.165) (end 148.615 73.165) (width 0.25) (layer F.Cu) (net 5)))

